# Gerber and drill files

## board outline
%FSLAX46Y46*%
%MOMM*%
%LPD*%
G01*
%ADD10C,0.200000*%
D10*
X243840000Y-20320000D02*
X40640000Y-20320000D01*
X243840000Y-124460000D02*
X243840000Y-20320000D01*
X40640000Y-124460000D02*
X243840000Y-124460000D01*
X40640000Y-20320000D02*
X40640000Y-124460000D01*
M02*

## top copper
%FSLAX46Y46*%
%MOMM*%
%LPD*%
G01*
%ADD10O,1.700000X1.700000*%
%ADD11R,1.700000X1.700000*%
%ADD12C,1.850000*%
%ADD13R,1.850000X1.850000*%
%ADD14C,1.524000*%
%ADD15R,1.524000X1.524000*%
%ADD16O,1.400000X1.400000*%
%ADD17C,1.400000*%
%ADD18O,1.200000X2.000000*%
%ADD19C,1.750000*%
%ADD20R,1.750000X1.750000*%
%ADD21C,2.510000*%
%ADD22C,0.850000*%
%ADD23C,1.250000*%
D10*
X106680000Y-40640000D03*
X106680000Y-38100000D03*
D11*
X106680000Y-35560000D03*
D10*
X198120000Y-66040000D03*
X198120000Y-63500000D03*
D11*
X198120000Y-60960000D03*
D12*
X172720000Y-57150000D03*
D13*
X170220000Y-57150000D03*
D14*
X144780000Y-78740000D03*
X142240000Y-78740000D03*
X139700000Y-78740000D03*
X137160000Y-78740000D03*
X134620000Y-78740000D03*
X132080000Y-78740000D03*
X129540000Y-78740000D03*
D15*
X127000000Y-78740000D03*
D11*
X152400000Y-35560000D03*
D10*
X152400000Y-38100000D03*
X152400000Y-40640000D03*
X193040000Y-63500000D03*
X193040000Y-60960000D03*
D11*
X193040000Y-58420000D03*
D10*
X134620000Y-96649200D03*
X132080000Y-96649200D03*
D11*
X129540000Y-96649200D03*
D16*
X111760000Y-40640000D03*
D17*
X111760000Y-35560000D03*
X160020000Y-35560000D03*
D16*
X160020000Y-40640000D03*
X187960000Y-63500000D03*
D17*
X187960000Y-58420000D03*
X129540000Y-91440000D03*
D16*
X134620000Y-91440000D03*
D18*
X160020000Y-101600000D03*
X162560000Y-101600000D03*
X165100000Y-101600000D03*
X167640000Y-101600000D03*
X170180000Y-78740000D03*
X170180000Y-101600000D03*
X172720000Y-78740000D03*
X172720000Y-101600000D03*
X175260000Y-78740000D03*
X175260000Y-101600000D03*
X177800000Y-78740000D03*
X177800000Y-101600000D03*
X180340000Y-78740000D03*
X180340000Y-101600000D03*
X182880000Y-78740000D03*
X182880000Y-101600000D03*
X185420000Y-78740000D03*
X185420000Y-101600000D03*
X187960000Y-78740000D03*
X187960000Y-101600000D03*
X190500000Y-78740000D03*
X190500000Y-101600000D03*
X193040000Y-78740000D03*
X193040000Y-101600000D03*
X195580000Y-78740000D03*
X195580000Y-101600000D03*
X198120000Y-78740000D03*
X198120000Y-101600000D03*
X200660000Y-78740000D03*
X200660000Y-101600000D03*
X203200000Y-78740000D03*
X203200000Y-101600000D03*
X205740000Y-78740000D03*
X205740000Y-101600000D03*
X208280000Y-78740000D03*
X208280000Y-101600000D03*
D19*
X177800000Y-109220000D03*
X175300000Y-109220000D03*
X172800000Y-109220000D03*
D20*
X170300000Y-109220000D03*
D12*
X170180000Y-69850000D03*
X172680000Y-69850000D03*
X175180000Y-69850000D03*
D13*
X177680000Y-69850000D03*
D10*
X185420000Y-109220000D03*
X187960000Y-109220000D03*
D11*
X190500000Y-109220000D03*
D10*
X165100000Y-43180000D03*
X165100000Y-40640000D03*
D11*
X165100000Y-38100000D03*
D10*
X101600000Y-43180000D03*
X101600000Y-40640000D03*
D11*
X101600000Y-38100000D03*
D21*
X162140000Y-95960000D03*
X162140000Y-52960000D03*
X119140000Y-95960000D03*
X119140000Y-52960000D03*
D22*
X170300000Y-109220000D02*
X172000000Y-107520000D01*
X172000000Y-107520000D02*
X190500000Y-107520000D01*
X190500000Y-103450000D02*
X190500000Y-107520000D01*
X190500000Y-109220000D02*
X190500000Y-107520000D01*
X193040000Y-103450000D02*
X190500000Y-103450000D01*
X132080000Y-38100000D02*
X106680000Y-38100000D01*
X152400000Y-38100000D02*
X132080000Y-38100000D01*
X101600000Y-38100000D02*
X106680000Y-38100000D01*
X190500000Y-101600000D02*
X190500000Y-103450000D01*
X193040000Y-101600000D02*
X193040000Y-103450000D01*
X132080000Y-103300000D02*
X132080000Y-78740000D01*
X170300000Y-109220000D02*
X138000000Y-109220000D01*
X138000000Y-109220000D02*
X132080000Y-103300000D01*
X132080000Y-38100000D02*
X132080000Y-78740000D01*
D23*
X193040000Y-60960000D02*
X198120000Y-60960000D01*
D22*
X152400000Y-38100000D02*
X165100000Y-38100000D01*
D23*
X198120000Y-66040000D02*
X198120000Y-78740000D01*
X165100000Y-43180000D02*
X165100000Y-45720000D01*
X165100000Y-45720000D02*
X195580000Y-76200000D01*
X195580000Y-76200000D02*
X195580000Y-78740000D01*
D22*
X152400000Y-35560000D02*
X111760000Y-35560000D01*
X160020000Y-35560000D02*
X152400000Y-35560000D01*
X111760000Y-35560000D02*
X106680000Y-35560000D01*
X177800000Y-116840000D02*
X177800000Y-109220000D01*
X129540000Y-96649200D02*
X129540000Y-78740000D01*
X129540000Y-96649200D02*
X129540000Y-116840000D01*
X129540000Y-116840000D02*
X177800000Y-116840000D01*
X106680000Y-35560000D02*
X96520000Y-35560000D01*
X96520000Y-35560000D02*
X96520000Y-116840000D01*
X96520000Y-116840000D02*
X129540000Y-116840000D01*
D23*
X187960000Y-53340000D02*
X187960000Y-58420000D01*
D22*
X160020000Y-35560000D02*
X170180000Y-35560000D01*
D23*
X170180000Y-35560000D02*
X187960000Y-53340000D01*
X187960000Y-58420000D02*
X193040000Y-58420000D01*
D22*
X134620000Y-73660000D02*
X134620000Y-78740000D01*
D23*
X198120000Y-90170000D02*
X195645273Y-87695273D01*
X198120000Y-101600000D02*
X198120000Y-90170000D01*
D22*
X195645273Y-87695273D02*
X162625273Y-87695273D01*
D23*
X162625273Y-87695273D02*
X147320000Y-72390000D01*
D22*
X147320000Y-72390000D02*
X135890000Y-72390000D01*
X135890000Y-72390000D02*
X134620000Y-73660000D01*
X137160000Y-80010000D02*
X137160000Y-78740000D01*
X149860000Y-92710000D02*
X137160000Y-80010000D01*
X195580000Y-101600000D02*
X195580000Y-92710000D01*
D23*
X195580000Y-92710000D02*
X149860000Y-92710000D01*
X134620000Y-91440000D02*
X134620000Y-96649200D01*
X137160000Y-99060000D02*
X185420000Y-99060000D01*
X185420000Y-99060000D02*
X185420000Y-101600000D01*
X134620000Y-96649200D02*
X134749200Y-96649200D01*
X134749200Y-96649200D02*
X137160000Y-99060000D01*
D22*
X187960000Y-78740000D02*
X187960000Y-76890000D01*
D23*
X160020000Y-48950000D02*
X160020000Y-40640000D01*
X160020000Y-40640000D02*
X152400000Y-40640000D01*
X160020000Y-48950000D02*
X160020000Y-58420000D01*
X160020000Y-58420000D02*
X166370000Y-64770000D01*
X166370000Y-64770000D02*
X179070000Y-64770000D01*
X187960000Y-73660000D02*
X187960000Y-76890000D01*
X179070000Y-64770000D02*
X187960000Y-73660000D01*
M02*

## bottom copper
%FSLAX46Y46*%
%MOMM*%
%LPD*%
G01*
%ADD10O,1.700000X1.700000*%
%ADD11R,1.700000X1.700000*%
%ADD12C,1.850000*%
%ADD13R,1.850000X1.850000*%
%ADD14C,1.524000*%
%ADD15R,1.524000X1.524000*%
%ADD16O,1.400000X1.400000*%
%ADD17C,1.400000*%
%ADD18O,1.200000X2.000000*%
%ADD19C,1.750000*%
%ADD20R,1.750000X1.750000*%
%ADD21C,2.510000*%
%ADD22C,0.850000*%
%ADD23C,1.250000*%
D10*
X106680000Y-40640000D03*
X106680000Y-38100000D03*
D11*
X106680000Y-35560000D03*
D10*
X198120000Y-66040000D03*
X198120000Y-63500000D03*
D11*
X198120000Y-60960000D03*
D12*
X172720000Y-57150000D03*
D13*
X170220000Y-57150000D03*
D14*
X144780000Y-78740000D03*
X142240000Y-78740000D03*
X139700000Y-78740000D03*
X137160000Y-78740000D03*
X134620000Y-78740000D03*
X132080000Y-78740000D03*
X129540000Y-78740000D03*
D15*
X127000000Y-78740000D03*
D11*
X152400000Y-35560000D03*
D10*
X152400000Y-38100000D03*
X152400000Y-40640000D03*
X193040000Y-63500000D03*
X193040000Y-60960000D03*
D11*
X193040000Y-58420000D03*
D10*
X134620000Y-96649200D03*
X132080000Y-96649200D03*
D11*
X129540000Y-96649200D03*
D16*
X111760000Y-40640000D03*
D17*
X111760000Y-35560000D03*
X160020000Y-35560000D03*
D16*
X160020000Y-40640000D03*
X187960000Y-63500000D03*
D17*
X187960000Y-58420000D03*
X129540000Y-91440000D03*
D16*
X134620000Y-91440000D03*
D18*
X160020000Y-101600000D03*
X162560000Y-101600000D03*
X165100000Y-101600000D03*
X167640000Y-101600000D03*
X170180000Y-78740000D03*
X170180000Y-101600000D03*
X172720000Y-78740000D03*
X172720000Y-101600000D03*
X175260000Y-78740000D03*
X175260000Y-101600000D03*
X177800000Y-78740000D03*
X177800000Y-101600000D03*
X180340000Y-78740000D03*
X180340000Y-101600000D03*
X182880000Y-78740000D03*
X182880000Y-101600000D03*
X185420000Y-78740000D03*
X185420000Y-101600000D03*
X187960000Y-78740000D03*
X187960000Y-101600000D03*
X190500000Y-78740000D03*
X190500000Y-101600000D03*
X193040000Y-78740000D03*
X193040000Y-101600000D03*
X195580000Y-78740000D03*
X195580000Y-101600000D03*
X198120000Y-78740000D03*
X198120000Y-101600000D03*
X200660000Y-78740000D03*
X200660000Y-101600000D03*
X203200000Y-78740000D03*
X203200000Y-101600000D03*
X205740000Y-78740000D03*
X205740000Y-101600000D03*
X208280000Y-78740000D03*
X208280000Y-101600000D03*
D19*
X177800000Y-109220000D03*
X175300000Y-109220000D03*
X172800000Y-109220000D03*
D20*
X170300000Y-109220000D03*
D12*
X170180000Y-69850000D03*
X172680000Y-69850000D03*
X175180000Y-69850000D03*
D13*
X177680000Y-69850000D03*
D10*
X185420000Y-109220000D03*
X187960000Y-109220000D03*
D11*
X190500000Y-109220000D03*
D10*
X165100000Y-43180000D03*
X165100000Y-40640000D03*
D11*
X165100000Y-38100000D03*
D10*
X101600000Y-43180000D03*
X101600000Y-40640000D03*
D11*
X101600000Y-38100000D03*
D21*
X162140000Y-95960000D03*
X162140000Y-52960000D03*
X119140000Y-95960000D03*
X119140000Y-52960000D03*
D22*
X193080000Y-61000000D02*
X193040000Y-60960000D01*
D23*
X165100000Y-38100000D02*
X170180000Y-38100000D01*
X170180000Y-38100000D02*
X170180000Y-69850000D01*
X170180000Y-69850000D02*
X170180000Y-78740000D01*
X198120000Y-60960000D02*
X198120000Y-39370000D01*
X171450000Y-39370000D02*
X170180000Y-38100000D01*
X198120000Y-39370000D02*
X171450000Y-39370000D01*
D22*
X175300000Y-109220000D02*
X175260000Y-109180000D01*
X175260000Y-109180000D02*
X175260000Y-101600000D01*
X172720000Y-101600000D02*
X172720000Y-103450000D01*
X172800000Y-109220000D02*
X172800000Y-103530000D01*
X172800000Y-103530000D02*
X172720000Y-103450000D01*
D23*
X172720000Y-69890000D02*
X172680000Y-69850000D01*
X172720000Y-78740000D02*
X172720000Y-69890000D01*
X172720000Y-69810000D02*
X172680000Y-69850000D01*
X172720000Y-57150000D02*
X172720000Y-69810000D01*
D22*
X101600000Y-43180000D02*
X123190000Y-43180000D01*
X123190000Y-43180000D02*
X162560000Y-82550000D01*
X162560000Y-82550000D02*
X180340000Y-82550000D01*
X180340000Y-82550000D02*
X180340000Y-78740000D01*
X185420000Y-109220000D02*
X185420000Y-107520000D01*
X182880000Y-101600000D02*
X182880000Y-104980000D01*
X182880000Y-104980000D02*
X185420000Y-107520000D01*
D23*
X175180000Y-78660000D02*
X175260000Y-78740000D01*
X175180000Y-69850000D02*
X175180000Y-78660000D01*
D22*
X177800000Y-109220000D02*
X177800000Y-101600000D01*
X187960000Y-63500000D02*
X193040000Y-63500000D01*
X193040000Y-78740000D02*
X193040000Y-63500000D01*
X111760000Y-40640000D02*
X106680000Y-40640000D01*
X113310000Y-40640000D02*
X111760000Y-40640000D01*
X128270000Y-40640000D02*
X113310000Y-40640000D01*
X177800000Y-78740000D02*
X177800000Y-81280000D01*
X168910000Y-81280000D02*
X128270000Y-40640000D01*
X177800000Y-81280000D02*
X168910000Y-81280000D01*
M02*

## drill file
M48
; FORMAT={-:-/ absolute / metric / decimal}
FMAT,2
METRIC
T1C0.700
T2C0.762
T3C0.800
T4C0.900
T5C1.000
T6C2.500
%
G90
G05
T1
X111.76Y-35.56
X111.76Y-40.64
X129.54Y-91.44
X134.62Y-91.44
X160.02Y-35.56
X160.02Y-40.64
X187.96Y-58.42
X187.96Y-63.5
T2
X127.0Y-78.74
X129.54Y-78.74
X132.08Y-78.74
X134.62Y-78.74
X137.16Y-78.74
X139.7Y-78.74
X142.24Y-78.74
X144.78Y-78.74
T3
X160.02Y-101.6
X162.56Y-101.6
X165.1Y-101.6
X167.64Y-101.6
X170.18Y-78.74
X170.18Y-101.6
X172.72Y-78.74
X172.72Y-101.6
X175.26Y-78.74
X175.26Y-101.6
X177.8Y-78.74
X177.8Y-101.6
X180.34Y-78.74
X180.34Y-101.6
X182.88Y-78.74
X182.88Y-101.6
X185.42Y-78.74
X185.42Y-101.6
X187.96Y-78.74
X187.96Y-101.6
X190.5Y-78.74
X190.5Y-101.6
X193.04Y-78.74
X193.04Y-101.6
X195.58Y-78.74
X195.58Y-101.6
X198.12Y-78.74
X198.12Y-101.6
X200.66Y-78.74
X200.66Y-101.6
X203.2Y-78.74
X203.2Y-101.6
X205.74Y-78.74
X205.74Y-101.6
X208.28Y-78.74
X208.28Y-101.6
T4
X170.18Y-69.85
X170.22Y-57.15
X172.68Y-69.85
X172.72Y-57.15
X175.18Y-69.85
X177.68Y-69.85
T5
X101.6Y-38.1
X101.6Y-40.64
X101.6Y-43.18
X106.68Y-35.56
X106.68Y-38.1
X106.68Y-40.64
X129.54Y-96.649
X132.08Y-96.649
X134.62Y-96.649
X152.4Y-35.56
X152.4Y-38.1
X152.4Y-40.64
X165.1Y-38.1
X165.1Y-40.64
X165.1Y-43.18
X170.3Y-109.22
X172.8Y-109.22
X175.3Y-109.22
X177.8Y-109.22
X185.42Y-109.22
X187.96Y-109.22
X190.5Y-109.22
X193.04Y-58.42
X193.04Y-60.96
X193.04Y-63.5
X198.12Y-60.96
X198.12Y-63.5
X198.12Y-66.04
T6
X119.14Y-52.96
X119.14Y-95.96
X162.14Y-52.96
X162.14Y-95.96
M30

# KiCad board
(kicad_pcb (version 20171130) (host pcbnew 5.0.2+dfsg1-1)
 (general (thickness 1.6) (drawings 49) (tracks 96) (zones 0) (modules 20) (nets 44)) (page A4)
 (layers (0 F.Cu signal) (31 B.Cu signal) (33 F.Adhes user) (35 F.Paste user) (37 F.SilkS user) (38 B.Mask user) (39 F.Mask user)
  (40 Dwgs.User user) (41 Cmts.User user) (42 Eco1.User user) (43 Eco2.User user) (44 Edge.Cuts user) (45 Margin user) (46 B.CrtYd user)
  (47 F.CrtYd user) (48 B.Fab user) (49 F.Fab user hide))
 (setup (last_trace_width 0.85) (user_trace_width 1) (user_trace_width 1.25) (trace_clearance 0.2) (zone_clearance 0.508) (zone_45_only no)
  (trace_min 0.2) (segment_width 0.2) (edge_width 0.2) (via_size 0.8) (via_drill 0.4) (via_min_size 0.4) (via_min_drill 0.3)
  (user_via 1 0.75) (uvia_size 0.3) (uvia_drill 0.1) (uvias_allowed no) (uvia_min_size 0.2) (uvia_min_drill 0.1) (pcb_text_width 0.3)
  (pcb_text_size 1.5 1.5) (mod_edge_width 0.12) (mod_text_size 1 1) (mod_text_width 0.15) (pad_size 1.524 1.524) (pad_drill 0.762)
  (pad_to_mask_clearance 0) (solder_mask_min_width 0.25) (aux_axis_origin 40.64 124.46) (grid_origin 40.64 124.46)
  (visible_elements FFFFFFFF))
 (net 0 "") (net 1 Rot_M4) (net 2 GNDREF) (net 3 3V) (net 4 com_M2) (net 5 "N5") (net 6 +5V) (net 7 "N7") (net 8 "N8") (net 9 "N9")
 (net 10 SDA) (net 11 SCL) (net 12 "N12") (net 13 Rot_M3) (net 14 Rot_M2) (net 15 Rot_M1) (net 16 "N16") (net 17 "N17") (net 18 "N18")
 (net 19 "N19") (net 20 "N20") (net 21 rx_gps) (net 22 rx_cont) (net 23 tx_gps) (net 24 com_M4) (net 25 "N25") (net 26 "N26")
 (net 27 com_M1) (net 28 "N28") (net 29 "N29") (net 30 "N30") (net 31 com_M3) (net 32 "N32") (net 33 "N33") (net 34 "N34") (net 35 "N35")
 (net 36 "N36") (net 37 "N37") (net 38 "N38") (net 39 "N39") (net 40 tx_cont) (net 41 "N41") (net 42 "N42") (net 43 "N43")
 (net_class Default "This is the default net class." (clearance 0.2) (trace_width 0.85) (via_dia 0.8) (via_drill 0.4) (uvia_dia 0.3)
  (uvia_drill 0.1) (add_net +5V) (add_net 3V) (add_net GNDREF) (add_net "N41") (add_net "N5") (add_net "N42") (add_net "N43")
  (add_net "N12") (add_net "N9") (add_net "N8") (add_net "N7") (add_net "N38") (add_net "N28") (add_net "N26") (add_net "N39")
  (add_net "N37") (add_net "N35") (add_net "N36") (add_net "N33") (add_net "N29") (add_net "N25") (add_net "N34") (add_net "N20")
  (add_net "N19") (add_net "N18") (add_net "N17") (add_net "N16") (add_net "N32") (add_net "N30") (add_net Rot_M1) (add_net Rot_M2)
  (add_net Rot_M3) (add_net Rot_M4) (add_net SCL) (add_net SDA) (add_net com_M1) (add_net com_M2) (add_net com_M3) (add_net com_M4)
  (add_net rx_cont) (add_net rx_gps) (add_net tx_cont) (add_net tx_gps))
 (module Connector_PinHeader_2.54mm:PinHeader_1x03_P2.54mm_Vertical (layer F.Cu) (at 106.68 35.56)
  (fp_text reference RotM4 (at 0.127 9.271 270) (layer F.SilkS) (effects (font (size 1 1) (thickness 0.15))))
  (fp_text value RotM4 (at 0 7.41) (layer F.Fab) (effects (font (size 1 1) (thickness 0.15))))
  (pad 3 thru_hole oval (at 0 5.08) (size 1.7 1.7) (drill 1) (layers *.Cu *.Mask) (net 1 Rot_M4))
  (pad 2 thru_hole oval (at 0 2.54) (size 1.7 1.7) (drill 1) (layers *.Cu *.Mask) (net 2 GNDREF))
  (pad 1 thru_hole rect (at 0 0) (size 1.7 1.7) (drill 1) (layers *.Cu *.Mask) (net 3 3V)))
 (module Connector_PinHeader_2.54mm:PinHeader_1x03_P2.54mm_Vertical (layer F.Cu) (at 198.12 60.96)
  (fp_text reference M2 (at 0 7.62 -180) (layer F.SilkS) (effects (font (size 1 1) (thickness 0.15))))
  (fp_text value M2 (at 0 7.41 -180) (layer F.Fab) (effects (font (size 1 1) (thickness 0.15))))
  (pad 3 thru_hole oval (at 0 5.08) (size 1.7 1.7) (drill 1) (layers *.Cu *.Mask) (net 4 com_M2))
  (pad 2 thru_hole oval (at 0 2.54) (size 1.7 1.7) (drill 1) (layers *.Cu *.Mask) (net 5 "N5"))
  (pad 1 thru_hole rect (at 0 0) (size 1.7 1.7) (drill 1) (layers *.Cu *.Mask) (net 2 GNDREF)))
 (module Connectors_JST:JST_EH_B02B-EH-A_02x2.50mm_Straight (layer F.Cu) (at 170.22 57.15)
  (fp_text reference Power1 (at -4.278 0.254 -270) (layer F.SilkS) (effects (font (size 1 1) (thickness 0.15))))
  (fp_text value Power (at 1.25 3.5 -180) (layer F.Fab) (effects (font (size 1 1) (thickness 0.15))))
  (pad 2 thru_hole circle (at 2.5 0) (size 1.85 1.85) (drill 0.9) (layers *.Cu *.Mask) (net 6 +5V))
  (pad 1 thru_hole rect (at 0 0) (size 1.85 1.85) (drill 0.9) (layers *.Cu *.Mask) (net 2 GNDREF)))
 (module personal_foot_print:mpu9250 (layer F.Cu) (at 132.08 76.2)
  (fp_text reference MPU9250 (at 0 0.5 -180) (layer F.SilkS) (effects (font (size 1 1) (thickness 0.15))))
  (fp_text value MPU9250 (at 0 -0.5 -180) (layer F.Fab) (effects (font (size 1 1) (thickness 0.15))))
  (pad 8 thru_hole circle (at 12.7 2.54) (size 1.524 1.524) (drill 0.762) (layers *.Cu *.Mask) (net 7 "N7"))
  (pad 7 thru_hole circle (at 10.16 2.54) (size 1.524 1.524) (drill 0.762) (layers *.Cu *.Mask) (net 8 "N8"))
  (pad 6 thru_hole circle (at 7.62 2.54) (size 1.524 1.524) (drill 0.762) (layers *.Cu *.Mask) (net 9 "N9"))
  (pad 5 thru_hole circle (at 5.08 2.54) (size 1.524 1.524) (drill 0.762) (layers *.Cu *.Mask) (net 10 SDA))
  (pad 4 thru_hole circle (at 2.54 2.54) (size 1.524 1.524) (drill 0.762) (layers *.Cu *.Mask) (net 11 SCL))
  (pad 3 thru_hole circle (at 0 2.54) (size 1.524 1.524) (drill 0.762) (layers *.Cu *.Mask) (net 2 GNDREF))
  (pad 2 thru_hole circle (at -2.54 2.54) (size 1.524 1.524) (drill 0.762) (layers *.Cu *.Mask) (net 3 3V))
  (pad 1 thru_hole rect (at -5.08 2.54) (size 1.524 1.524) (drill 0.762) (layers *.Cu *.Mask) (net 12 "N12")))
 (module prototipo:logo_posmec (layer F.Cu) (at 235.077 42.469 90)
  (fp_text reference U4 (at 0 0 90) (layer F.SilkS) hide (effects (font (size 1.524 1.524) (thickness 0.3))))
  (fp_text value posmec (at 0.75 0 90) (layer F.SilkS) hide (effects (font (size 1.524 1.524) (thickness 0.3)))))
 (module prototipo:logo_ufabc (layer F.Cu) (at 54.61 53.645 90)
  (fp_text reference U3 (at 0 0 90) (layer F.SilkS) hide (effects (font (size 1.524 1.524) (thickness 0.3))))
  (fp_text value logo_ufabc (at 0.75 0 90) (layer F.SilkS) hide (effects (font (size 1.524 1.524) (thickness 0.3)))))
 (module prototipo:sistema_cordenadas (layer F.Cu) (at 140.843 80.95 270)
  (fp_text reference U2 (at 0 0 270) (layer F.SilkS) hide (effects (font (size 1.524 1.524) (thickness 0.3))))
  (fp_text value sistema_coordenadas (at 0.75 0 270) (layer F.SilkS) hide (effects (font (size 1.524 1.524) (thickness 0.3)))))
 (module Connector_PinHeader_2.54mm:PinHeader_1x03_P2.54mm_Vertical (layer F.Cu) (at 152.4 35.56)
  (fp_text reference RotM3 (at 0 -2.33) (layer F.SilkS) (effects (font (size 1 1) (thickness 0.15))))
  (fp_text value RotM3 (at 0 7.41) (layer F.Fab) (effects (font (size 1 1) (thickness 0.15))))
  (pad 1 thru_hole rect (at 0 0) (size 1.7 1.7) (drill 1) (layers *.Cu *.Mask) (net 3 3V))
  (pad 2 thru_hole oval (at 0 2.54) (size 1.7 1.7) (drill 1) (layers *.Cu *.Mask) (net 2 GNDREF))
  (pad 3 thru_hole oval (at 0 5.08) (size 1.7 1.7) (drill 1) (layers *.Cu *.Mask) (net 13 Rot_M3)))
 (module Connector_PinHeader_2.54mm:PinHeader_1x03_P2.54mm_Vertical (layer F.Cu) (at 193.04 58.42)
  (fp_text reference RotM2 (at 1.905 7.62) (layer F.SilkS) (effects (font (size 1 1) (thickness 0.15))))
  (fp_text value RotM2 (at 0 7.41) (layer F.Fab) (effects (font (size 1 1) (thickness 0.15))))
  (pad 3 thru_hole oval (at 0 5.08) (size 1.7 1.7) (drill 1) (layers *.Cu *.Mask) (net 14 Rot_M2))
  (pad 2 thru_hole oval (at 0 2.54) (size 1.7 1.7) (drill 1) (layers *.Cu *.Mask) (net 2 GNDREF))
  (pad 1 thru_hole rect (at 0 0) (size 1.7 1.7) (drill 1) (layers *.Cu *.Mask) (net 3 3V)))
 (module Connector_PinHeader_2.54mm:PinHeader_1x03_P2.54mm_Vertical (layer F.Cu) (at 129.54 96.6492 90)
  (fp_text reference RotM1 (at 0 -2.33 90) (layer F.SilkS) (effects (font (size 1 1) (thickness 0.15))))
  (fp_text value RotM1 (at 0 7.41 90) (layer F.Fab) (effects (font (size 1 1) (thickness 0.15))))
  (pad 3 thru_hole oval (at 0 5.08 90) (size 1.7 1.7) (drill 1) (layers *.Cu *.Mask) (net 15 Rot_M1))
  (pad 2 thru_hole oval (at 0 2.54 90) (size 1.7 1.7) (drill 1) (layers *.Cu *.Mask) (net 2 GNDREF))
  (pad 1 thru_hole rect (at 0 0 90) (size 1.7 1.7) (drill 1) (layers *.Cu *.Mask) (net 3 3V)))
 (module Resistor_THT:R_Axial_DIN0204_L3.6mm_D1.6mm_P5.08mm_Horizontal (layer F.Cu) (at 111.76 35.56 270)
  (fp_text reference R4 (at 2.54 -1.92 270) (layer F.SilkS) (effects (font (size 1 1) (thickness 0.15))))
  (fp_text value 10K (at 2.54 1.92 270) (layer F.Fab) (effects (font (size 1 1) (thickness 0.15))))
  (pad 2 thru_hole oval (at 5.08 0 270) (size 1.4 1.4) (drill 0.7) (layers *.Cu *.Mask) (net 1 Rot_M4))
  (pad 1 thru_hole circle (at 0 0 270) (size 1.4 1.4) (drill 0.7) (layers *.Cu *.Mask) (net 3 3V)))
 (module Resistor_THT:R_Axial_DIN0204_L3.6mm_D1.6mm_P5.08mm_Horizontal (layer F.Cu) (at 160.02 35.56 270)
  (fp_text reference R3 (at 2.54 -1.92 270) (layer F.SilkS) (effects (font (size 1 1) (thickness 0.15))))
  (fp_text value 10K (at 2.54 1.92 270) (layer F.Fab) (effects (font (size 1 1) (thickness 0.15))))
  (pad 1 thru_hole circle (at 0 0 270) (size 1.4 1.4) (drill 0.7) (layers *.Cu *.Mask) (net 3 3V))
  (pad 2 thru_hole oval (at 5.08 0 270) (size 1.4 1.4) (drill 0.7) (layers *.Cu *.Mask) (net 13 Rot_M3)))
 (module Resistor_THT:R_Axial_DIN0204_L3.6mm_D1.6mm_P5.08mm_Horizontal (layer F.Cu) (at 187.96 58.42 270)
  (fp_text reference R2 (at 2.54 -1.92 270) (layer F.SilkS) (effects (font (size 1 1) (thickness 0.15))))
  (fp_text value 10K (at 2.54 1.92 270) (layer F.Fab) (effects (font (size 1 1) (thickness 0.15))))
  (pad 2 thru_hole oval (at 5.08 0 270) (size 1.4 1.4) (drill 0.7) (layers *.Cu *.Mask) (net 14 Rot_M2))
  (pad 1 thru_hole circle (at 0 0 270) (size 1.4 1.4) (drill 0.7) (layers *.Cu *.Mask) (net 3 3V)))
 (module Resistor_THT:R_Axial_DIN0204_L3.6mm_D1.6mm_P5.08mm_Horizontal (layer F.Cu) (at 129.54 91.44)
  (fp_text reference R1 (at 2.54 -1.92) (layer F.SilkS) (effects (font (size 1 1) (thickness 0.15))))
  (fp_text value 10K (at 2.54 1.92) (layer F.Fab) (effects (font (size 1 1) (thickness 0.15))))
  (pad 1 thru_hole circle (at 0 0) (size 1.4 1.4) (drill 0.7) (layers *.Cu *.Mask) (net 3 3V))
  (pad 2 thru_hole oval (at 5.08 0) (size 1.4 1.4) (drill 0.7) (layers *.Cu *.Mask) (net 15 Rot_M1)))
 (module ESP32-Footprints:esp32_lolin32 (layer F.Cu) (at 189.23 90.17 270)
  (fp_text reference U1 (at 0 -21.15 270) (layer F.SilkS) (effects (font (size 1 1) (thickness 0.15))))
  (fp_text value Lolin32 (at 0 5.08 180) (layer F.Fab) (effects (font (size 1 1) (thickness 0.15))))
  (pad 36 thru_hole oval (at 11.43 29.21 180) (size 1.2 2) (drill 0.8) (layers *.Cu *.Mask) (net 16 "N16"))
  (pad 35 thru_hole oval (at 11.43 26.67 180) (size 1.2 2) (drill 0.8) (layers *.Cu *.Mask) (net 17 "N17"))
  (pad 34 thru_hole oval (at 11.43 24.13 180) (size 1.2 2) (drill 0.8) (layers *.Cu *.Mask) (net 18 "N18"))
  (pad 33 thru_hole oval (at 11.43 21.59 180) (size 1.2 2) (drill 0.8) (layers *.Cu *.Mask) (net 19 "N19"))
  (pad 16 thru_hole oval (at -11.43 19.05 180) (size 1.2 2) (drill 0.8) (layers *.Cu *.Mask) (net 2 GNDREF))
  (pad 32 thru_hole oval (at 11.43 19.05 180) (size 1.2 2) (drill 0.8) (layers *.Cu *.Mask) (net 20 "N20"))
  (pad 15 thru_hole oval (at -11.43 16.51 180) (size 1.2 2) (drill 0.8) (layers *.Cu *.Mask) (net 6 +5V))
  (pad 31 thru_hole oval (at 11.43 16.51 180) (size 1.2 2) (drill 0.8) (layers *.Cu *.Mask) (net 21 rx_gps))
  (pad 14 thru_hole oval (at -11.43 13.97 180) (size 1.2 2) (drill 0.8) (layers *.Cu *.Mask) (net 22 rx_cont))
  (pad 30 thru_hole oval (at 11.43 13.97 180) (size 1.2 2) (drill 0.8) (layers *.Cu *.Mask) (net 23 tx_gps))
  (pad 13 thru_hole oval (at -11.43 11.43 180) (size 1.2 2) (drill 0.8) (layers *.Cu *.Mask) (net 1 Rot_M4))
  (pad 29 thru_hole oval (at 11.43 11.43 180) (size 1.2 2) (drill 0.8) (layers *.Cu *.Mask) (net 3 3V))
  (pad 12 thru_hole oval (at -11.43 8.89 180) (size 1.2 2) (drill 0.8) (layers *.Cu *.Mask) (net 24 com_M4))
  (pad 28 thru_hole oval (at 11.43 8.89 180) (size 1.2 2) (drill 0.8) (layers *.Cu *.Mask) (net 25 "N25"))
  (pad 11 thru_hole oval (at -11.43 6.35 180) (size 1.2 2) (drill 0.8) (layers *.Cu *.Mask) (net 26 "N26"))
  (pad 27 thru_hole oval (at 11.43 6.35 180) (size 1.2 2) (drill 0.8) (layers *.Cu *.Mask) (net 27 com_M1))
  (pad 10 thru_hole oval (at -11.43 3.81 180) (size 1.2 2) (drill 0.8) (layers *.Cu *.Mask) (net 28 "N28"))
  (pad 26 thru_hole oval (at 11.43 3.81 180) (size 1.2 2) (drill 0.8) (layers *.Cu *.Mask) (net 15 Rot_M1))
  (pad 9 thru_hole oval (at -11.43 1.27 180) (size 1.2 2) (drill 0.8) (layers *.Cu *.Mask) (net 13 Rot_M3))
  (pad 25 thru_hole oval (at 11.43 1.27 180) (size 1.2 2) (drill 0.8) (layers *.Cu *.Mask) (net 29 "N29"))
  (pad 8 thru_hole oval (at -11.43 -1.27 180) (size 1.2 2) (drill 0.8) (layers *.Cu *.Mask) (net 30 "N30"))
  (pad 24 thru_hole oval (at 11.43 -1.27 180) (size 1.2 2) (drill 0.8) (layers *.Cu *.Mask) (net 2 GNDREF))
  (pad 7 thru_hole oval (at -11.43 -3.81 180) (size 1.2 2) (drill 0.8) (layers *.Cu *.Mask) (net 14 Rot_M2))
  (pad 23 thru_hole oval (at 11.43 -3.81 180) (size 1.2 2) (drill 0.8) (layers *.Cu *.Mask) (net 2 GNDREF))
  (pad 6 thru_hole oval (at -11.43 -6.35 180) (size 1.2 2) (drill 0.8) (layers *.Cu *.Mask) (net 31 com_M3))
  (pad 22 thru_hole oval (at 11.43 -6.35 180) (size 1.2 2) (drill 0.8) (layers *.Cu *.Mask) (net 10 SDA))
  (pad 5 thru_hole oval (at -11.43 -8.89 180) (size 1.2 2) (drill 0.8) (layers *.Cu *.Mask) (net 4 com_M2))
  (pad 21 thru_hole oval (at 11.43 -8.89 180) (size 1.2 2) (drill 0.8) (layers *.Cu *.Mask) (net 11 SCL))
  (pad 4 thru_hole oval (at -11.43 -11.43 180) (size 1.2 2) (drill 0.8) (layers *.Cu *.Mask) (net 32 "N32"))
  (pad 20 thru_hole oval (at 11.43 -11.43 180) (size 1.2 2) (drill 0.8) (layers *.Cu *.Mask) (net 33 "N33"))
  (pad 3 thru_hole oval (at -11.43 -13.97 180) (size 1.2 2) (drill 0.8) (layers *.Cu *.Mask) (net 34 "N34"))
  (pad 19 thru_hole oval (at 11.43 -13.97 180) (size 1.2 2) (drill 0.8) (layers *.Cu *.Mask) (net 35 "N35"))
  (pad 2 thru_hole oval (at -11.43 -16.51 180) (size 1.2 2) (drill 0.8) (layers *.Cu *.Mask) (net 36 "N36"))
  (pad 18 thru_hole oval (at 11.43 -16.51 180) (size 1.2 2) (drill 0.8) (layers *.Cu *.Mask) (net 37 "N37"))
  (pad 1 thru_hole oval (at -11.43 -19.05 180) (size 1.2 2) (drill 0.8) (layers *.Cu *.Mask) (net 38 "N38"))
  (pad 17 thru_hole oval (at 11.43 -19.05 180) (size 1.2 2) (drill 0.8) (layers *.Cu *.Mask) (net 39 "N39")))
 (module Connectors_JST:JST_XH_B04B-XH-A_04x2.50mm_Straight (layer F.Cu) (at 170.3 109.22)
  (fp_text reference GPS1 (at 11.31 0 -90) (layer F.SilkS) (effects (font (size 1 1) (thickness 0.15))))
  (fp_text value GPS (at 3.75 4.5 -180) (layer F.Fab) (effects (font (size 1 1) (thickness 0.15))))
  (pad 4 thru_hole circle (at 7.5 0) (size 1.75 1.75) (drill 1) (layers *.Cu *.Mask) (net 3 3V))
  (pad 3 thru_hole circle (at 5 0) (size 1.75 1.75) (drill 1) (layers *.Cu *.Mask) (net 23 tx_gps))
  (pad 2 thru_hole circle (at 2.5 0) (size 1.75 1.75) (drill 1) (layers *.Cu *.Mask) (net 21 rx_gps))
  (pad 1 thru_hole rect (at 0 0) (size 1.75 1.75) (drill 1) (layers *.Cu *.Mask) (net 2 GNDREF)))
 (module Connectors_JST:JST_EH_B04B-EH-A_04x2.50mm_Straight (layer F.Cu) (at 177.68 69.85 180)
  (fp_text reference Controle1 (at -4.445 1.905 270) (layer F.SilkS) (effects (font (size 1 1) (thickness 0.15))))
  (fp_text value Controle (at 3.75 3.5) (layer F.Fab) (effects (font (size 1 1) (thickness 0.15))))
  (pad 4 thru_hole circle (at 7.5 0 180) (size 1.85 1.85) (drill 0.9) (layers *.Cu *.Mask) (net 2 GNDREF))
  (pad 3 thru_hole circle (at 5 0 180) (size 1.85 1.85) (drill 0.9) (layers *.Cu *.Mask) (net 6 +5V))
  (pad 2 thru_hole circle (at 2.5 0 180) (size 1.85 1.85) (drill 0.9) (layers *.Cu *.Mask) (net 22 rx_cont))
  (pad 1 thru_hole rect (at 0 0 180) (size 1.85 1.85) (drill 0.9) (layers *.Cu *.Mask) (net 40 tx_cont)))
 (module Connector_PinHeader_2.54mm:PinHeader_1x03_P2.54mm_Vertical (layer F.Cu) (at 190.5 109.22 270)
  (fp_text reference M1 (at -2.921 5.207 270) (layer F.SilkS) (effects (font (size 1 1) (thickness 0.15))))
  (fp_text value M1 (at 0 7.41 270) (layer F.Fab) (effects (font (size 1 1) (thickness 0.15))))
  (pad 3 thru_hole oval (at 0 5.08 270) (size 1.7 1.7) (drill 1) (layers *.Cu *.Mask) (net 27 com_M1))
  (pad 2 thru_hole oval (at 0 2.54 270) (size 1.7 1.7) (drill 1) (layers *.Cu *.Mask) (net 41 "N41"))
  (pad 1 thru_hole rect (at 0 0 270) (size 1.7 1.7) (drill 1) (layers *.Cu *.Mask) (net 2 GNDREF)))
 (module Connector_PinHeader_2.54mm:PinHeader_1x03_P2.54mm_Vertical (layer F.Cu) (at 165.1 38.1)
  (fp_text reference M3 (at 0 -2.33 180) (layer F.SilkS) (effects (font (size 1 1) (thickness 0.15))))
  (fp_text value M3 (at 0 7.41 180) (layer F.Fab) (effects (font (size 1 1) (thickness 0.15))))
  (pad 3 thru_hole oval (at 0 5.08) (size 1.7 1.7) (drill 1) (layers *.Cu *.Mask) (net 31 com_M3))
  (pad 2 thru_hole oval (at 0 2.54) (size 1.7 1.7) (drill 1) (layers *.Cu *.Mask) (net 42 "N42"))
  (pad 1 thru_hole rect (at 0 0) (size 1.7 1.7) (drill 1) (layers *.Cu *.Mask) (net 2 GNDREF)))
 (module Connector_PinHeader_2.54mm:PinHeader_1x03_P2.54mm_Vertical (layer F.Cu) (at 101.6 38.1)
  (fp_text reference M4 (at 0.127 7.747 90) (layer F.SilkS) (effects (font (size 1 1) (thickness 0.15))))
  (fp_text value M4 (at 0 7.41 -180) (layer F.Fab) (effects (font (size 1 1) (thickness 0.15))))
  (pad 3 thru_hole oval (at 0 5.08) (size 1.7 1.7) (drill 1) (layers *.Cu *.Mask) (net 24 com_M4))
  (pad 2 thru_hole oval (at 0 2.54) (size 1.7 1.7) (drill 1) (layers *.Cu *.Mask) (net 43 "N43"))
  (pad 1 thru_hole rect (at 0 0) (size 1.7 1.7) (drill 1) (layers *.Cu *.Mask) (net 2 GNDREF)))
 (gr_line (start 243.84 20.32) (end 40.64 20.32) (layer Edge.Cuts) (width 0.2))
 (gr_line (start 243.84 124.46) (end 243.84 20.32) (layer Edge.Cuts) (width 0.2))
 (gr_line (start 40.64 124.46) (end 243.84 124.46) (layer Edge.Cuts) (width 0.2))
 (gr_line (start 40.64 20.32) (end 40.64 124.46) (layer Edge.Cuts) (width 0.2))
 (via (at 162.14 95.96) (size 2.51) (drill 2.5) (layers F.Cu B.Cu) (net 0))
 (via (at 162.14 52.96) (size 2.51) (drill 2.5) (layers F.Cu B.Cu) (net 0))
 (via (at 119.14 95.96) (size 2.51) (drill 2.5) (layers F.Cu B.Cu) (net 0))
 (via (at 119.14 52.96) (size 2.51) (drill 2.5) (layers F.Cu B.Cu) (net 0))
 (segment (start 170.3 109.22) (end 172 107.52) (width 0.85) (layer F.Cu) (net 2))
 (segment (start 172 107.52) (end 190.5 107.52) (width 0.85) (layer F.Cu) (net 2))
 (segment (start 190.5 103.45) (end 190.5 107.52) (width 0.85) (layer F.Cu) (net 2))
 (segment (start 190.5 109.22) (end 190.5 107.52) (width 0.85) (layer F.Cu) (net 2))
 (segment (start 193.04 103.45) (end 190.5 103.45) (width 0.85) (layer F.Cu) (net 2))
 (segment (start 132.08 38.1) (end 106.68 38.1) (width 0.85) (layer F.Cu) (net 2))
 (segment (start 152.4 38.1) (end 132.08 38.1) (width 0.85) (layer F.Cu) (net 2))
 (segment (start 101.6 38.1) (end 106.68 38.1) (width 0.85) (layer F.Cu) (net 2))
 (segment (start 190.5 101.6) (end 190.5 103.45) (width 0.85) (layer F.Cu) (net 2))
 (segment (start 193.04 101.6) (end 193.04 103.45) (width 0.85) (layer F.Cu) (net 2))
 (segment (start 132.08 103.3) (end 132.08 78.74) (width 0.85) (layer F.Cu) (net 2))
 (segment (start 170.3 109.22) (end 138 109.22) (width 0.85) (layer F.Cu) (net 2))
 (segment (start 138 109.22) (end 132.08 103.3) (width 0.85) (layer F.Cu) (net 2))
 (segment (start 132.08 38.1) (end 132.08 78.74) (width 0.85) (layer F.Cu) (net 2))
 (segment (start 193.08 61) (end 193.04 60.96) (width 0.85) (layer B.Cu) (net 2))
 (segment (start 193.04 60.96) (end 198.12 60.96) (width 1.25) (layer F.Cu) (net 2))
 (segment (start 152.4 38.1) (end 165.1 38.1) (width 0.85) (layer F.Cu) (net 2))
 (segment (start 165.1 38.1) (end 170.18 38.1) (width 1.25) (layer B.Cu) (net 2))
 (segment (start 170.18 38.1) (end 170.18 69.85) (width 1.25) (layer B.Cu) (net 2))
 (segment (start 170.18 69.85) (end 170.18 78.74) (width 1.25) (layer B.Cu) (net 2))
 (segment (start 198.12 60.96) (end 198.12 39.37) (width 1.25) (layer B.Cu) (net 2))
 (segment (start 171.45 39.37) (end 170.18 38.1) (width 1.25) (layer B.Cu) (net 2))
 (segment (start 198.12 39.37) (end 171.45 39.37) (width 1.25) (layer B.Cu) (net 2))
 (segment (start 175.3 109.22) (end 175.26 109.18) (width 0.85) (layer B.Cu) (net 23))
 (segment (start 175.26 109.18) (end 175.26 101.6) (width 0.85) (layer B.Cu) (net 23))
 (segment (start 172.72 101.6) (end 172.72 103.45) (width 0.85) (layer B.Cu) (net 21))
 (segment (start 172.8 109.22) (end 172.8 103.53) (width 0.85) (layer B.Cu) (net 21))
 (segment (start 172.8 103.53) (end 172.72 103.45) (width 0.85) (layer B.Cu) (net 21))
 (segment (start 172.72 69.89) (end 172.68 69.85) (width 1.25) (layer B.Cu) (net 6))
 (segment (start 172.72 78.74) (end 172.72 69.89) (width 1.25) (layer B.Cu) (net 6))
 (segment (start 172.72 69.81) (end 172.68 69.85) (width 1.25) (layer B.Cu) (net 6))
 (segment (start 172.72 57.15) (end 172.72 69.81) (width 1.25) (layer B.Cu) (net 6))
 (segment (start 101.6 43.18) (end 123.19 43.18) (width 0.85) (layer B.Cu) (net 24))
 (segment (start 123.19 43.18) (end 162.56 82.55) (width 0.85) (layer B.Cu) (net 24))
 (segment (start 162.56 82.55) (end 180.34 82.55) (width 0.85) (layer B.Cu) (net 24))
 (segment (start 180.34 82.55) (end 180.34 78.74) (width 0.85) (layer B.Cu) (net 24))
 (segment (start 198.12 66.04) (end 198.12 78.74) (width 1.25) (layer F.Cu) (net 4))
 (segment (start 165.1 43.18) (end 165.1 45.72) (width 1.25) (layer F.Cu) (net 31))
 (segment (start 165.1 45.72) (end 195.58 76.2) (width 1.25) (layer F.Cu) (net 31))
 (segment (start 195.58 76.2) (end 195.58 78.74) (width 1.25) (layer F.Cu) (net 31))
 (segment (start 185.42 109.22) (end 185.42 107.52) (width 0.85) (layer B.Cu) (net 27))
 (segment (start 182.88 101.6) (end 182.88 104.98) (width 0.85) (layer B.Cu) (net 27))
 (segment (start 182.88 104.98) (end 185.42 107.52) (width 0.85) (layer B.Cu) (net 27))
 (segment (start 175.18 78.66) (end 175.26 78.74) (width 1.25) (layer B.Cu) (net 22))
 (segment (start 175.18 69.85) (end 175.18 78.66) (width 1.25) (layer B.Cu) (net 22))
 (segment (start 152.4 35.56) (end 111.76 35.56) (width 0.85) (layer F.Cu) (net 3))
 (segment (start 160.02 35.56) (end 152.4 35.56) (width 0.85) (layer F.Cu) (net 3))
 (segment (start 111.76 35.56) (end 106.68 35.56) (width 0.85) (layer F.Cu) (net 3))
 (segment (start 177.8 109.22) (end 177.8 101.6) (width 0.85) (layer B.Cu) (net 3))
 (segment (start 177.8 116.84) (end 177.8 109.22) (width 0.85) (layer F.Cu) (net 3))
 (segment (start 129.54 96.6492) (end 129.54 78.74) (width 0.85) (layer F.Cu) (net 3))
 (segment (start 129.54 96.6492) (end 129.54 116.84) (width 0.85) (layer F.Cu) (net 3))
 (segment (start 129.54 116.84) (end 177.8 116.84) (width 0.85) (layer F.Cu) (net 3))
 (segment (start 106.68 35.56) (end 96.52 35.56) (width 0.85) (layer F.Cu) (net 3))
 (segment (start 96.52 35.56) (end 96.52 116.84) (width 0.85) (layer F.Cu) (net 3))
 (segment (start 96.52 116.84) (end 129.54 116.84) (width 0.85) (layer F.Cu) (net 3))
 (segment (start 187.96 53.34) (end 187.96 58.42) (width 1.25) (layer F.Cu) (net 3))
 (segment (start 160.02 35.56) (end 170.18 35.56) (width 0.85) (layer F.Cu) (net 3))
 (segment (start 170.18 35.56) (end 187.96 53.34) (width 1.25) (layer F.Cu) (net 3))
 (segment (start 187.96 58.42) (end 193.04 58.42) (width 1.25) (layer F.Cu) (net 3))
 (segment (start 134.62 73.66) (end 134.62 78.74) (width 0.85) (layer F.Cu) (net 11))
 (segment (start 198.12 90.17) (end 195.645273 87.695273) (width 1.25) (layer F.Cu) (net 11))
 (segment (start 198.12 101.6) (end 198.12 90.17) (width 1.25) (layer F.Cu) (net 11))
 (segment (start 195.645273 87.695273) (end 162.625273 87.695273) (width 0.85) (layer F.Cu) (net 11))
 (segment (start 162.625273 87.695273) (end 147.32 72.39) (width 1.25) (layer F.Cu) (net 11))
 (segment (start 147.32 72.39) (end 135.89 72.39) (width 0.85) (layer F.Cu) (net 11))
 (segment (start 135.89 72.39) (end 134.62 73.66) (width 0.85) (layer F.Cu) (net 11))
 (segment (start 137.16 80.01) (end 137.16 78.74) (width 0.85) (layer F.Cu) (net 10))
 (segment (start 149.86 92.71) (end 137.16 80.01) (width 0.85) (layer F.Cu) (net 10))
 (segment (start 195.58 101.6) (end 195.58 92.71) (width 0.85) (layer F.Cu) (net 10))
 (segment (start 195.58 92.71) (end 149.86 92.71) (width 1.25) (layer F.Cu) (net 10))
 (segment (start 187.96 63.5) (end 193.04 63.5) (width 0.85) (layer B.Cu) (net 14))
 (segment (start 193.04 78.74) (end 193.04 63.5) (width 0.85) (layer B.Cu) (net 14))
 (segment (start 134.62 91.44) (end 134.62 96.6492) (width 1.25) (layer F.Cu) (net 15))
 (segment (start 137.16 99.06) (end 185.42 99.06) (width 1.25) (layer F.Cu) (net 15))
 (segment (start 185.42 99.06) (end 185.42 101.6) (width 1.25) (layer F.Cu) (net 15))
 (segment (start 134.62 96.6492) (end 134.7492 96.6492) (width 1.25) (layer F.Cu) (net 15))
 (segment (start 134.7492 96.6492) (end 137.16 99.06) (width 1.25) (layer F.Cu) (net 15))
 (segment (start 187.96 78.74) (end 187.96 76.89) (width 0.85) (layer F.Cu) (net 13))
 (segment (start 160.02 48.95) (end 160.02 40.64) (width 1.25) (layer F.Cu) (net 13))
 (segment (start 160.02 40.64) (end 152.4 40.64) (width 1.25) (layer F.Cu) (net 13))
 (segment (start 160.02 48.95) (end 160.02 58.42) (width 1.25) (layer F.Cu) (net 13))
 (segment (start 160.02 58.42) (end 166.37 64.77) (width 1.25) (layer F.Cu) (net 13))
 (segment (start 166.37 64.77) (end 179.07 64.77) (width 1.25) (layer F.Cu) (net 13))
 (segment (start 187.96 73.66) (end 187.96 76.89) (width 1.25) (layer F.Cu) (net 13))
 (segment (start 179.07 64.77) (end 187.96 73.66) (width 1.25) (layer F.Cu) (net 13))
 (segment (start 111.76 40.64) (end 106.68 40.64) (width 0.85) (layer B.Cu) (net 1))
 (segment (start 113.31 40.64) (end 111.76 40.64) (width 0.85) (layer B.Cu) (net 1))
 (segment (start 128.27 40.64) (end 113.31 40.64) (width 0.85) (layer B.Cu) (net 1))
 (segment (start 177.8 78.74) (end 177.8 81.28) (width 0.85) (layer B.Cu) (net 1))
 (segment (start 168.91 81.28) (end 128.27 40.64) (width 0.85) (layer B.Cu) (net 1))
 (segment (start 177.8 81.28) (end 168.91 81.28) (width 0.85) (layer B.Cu) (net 1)))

